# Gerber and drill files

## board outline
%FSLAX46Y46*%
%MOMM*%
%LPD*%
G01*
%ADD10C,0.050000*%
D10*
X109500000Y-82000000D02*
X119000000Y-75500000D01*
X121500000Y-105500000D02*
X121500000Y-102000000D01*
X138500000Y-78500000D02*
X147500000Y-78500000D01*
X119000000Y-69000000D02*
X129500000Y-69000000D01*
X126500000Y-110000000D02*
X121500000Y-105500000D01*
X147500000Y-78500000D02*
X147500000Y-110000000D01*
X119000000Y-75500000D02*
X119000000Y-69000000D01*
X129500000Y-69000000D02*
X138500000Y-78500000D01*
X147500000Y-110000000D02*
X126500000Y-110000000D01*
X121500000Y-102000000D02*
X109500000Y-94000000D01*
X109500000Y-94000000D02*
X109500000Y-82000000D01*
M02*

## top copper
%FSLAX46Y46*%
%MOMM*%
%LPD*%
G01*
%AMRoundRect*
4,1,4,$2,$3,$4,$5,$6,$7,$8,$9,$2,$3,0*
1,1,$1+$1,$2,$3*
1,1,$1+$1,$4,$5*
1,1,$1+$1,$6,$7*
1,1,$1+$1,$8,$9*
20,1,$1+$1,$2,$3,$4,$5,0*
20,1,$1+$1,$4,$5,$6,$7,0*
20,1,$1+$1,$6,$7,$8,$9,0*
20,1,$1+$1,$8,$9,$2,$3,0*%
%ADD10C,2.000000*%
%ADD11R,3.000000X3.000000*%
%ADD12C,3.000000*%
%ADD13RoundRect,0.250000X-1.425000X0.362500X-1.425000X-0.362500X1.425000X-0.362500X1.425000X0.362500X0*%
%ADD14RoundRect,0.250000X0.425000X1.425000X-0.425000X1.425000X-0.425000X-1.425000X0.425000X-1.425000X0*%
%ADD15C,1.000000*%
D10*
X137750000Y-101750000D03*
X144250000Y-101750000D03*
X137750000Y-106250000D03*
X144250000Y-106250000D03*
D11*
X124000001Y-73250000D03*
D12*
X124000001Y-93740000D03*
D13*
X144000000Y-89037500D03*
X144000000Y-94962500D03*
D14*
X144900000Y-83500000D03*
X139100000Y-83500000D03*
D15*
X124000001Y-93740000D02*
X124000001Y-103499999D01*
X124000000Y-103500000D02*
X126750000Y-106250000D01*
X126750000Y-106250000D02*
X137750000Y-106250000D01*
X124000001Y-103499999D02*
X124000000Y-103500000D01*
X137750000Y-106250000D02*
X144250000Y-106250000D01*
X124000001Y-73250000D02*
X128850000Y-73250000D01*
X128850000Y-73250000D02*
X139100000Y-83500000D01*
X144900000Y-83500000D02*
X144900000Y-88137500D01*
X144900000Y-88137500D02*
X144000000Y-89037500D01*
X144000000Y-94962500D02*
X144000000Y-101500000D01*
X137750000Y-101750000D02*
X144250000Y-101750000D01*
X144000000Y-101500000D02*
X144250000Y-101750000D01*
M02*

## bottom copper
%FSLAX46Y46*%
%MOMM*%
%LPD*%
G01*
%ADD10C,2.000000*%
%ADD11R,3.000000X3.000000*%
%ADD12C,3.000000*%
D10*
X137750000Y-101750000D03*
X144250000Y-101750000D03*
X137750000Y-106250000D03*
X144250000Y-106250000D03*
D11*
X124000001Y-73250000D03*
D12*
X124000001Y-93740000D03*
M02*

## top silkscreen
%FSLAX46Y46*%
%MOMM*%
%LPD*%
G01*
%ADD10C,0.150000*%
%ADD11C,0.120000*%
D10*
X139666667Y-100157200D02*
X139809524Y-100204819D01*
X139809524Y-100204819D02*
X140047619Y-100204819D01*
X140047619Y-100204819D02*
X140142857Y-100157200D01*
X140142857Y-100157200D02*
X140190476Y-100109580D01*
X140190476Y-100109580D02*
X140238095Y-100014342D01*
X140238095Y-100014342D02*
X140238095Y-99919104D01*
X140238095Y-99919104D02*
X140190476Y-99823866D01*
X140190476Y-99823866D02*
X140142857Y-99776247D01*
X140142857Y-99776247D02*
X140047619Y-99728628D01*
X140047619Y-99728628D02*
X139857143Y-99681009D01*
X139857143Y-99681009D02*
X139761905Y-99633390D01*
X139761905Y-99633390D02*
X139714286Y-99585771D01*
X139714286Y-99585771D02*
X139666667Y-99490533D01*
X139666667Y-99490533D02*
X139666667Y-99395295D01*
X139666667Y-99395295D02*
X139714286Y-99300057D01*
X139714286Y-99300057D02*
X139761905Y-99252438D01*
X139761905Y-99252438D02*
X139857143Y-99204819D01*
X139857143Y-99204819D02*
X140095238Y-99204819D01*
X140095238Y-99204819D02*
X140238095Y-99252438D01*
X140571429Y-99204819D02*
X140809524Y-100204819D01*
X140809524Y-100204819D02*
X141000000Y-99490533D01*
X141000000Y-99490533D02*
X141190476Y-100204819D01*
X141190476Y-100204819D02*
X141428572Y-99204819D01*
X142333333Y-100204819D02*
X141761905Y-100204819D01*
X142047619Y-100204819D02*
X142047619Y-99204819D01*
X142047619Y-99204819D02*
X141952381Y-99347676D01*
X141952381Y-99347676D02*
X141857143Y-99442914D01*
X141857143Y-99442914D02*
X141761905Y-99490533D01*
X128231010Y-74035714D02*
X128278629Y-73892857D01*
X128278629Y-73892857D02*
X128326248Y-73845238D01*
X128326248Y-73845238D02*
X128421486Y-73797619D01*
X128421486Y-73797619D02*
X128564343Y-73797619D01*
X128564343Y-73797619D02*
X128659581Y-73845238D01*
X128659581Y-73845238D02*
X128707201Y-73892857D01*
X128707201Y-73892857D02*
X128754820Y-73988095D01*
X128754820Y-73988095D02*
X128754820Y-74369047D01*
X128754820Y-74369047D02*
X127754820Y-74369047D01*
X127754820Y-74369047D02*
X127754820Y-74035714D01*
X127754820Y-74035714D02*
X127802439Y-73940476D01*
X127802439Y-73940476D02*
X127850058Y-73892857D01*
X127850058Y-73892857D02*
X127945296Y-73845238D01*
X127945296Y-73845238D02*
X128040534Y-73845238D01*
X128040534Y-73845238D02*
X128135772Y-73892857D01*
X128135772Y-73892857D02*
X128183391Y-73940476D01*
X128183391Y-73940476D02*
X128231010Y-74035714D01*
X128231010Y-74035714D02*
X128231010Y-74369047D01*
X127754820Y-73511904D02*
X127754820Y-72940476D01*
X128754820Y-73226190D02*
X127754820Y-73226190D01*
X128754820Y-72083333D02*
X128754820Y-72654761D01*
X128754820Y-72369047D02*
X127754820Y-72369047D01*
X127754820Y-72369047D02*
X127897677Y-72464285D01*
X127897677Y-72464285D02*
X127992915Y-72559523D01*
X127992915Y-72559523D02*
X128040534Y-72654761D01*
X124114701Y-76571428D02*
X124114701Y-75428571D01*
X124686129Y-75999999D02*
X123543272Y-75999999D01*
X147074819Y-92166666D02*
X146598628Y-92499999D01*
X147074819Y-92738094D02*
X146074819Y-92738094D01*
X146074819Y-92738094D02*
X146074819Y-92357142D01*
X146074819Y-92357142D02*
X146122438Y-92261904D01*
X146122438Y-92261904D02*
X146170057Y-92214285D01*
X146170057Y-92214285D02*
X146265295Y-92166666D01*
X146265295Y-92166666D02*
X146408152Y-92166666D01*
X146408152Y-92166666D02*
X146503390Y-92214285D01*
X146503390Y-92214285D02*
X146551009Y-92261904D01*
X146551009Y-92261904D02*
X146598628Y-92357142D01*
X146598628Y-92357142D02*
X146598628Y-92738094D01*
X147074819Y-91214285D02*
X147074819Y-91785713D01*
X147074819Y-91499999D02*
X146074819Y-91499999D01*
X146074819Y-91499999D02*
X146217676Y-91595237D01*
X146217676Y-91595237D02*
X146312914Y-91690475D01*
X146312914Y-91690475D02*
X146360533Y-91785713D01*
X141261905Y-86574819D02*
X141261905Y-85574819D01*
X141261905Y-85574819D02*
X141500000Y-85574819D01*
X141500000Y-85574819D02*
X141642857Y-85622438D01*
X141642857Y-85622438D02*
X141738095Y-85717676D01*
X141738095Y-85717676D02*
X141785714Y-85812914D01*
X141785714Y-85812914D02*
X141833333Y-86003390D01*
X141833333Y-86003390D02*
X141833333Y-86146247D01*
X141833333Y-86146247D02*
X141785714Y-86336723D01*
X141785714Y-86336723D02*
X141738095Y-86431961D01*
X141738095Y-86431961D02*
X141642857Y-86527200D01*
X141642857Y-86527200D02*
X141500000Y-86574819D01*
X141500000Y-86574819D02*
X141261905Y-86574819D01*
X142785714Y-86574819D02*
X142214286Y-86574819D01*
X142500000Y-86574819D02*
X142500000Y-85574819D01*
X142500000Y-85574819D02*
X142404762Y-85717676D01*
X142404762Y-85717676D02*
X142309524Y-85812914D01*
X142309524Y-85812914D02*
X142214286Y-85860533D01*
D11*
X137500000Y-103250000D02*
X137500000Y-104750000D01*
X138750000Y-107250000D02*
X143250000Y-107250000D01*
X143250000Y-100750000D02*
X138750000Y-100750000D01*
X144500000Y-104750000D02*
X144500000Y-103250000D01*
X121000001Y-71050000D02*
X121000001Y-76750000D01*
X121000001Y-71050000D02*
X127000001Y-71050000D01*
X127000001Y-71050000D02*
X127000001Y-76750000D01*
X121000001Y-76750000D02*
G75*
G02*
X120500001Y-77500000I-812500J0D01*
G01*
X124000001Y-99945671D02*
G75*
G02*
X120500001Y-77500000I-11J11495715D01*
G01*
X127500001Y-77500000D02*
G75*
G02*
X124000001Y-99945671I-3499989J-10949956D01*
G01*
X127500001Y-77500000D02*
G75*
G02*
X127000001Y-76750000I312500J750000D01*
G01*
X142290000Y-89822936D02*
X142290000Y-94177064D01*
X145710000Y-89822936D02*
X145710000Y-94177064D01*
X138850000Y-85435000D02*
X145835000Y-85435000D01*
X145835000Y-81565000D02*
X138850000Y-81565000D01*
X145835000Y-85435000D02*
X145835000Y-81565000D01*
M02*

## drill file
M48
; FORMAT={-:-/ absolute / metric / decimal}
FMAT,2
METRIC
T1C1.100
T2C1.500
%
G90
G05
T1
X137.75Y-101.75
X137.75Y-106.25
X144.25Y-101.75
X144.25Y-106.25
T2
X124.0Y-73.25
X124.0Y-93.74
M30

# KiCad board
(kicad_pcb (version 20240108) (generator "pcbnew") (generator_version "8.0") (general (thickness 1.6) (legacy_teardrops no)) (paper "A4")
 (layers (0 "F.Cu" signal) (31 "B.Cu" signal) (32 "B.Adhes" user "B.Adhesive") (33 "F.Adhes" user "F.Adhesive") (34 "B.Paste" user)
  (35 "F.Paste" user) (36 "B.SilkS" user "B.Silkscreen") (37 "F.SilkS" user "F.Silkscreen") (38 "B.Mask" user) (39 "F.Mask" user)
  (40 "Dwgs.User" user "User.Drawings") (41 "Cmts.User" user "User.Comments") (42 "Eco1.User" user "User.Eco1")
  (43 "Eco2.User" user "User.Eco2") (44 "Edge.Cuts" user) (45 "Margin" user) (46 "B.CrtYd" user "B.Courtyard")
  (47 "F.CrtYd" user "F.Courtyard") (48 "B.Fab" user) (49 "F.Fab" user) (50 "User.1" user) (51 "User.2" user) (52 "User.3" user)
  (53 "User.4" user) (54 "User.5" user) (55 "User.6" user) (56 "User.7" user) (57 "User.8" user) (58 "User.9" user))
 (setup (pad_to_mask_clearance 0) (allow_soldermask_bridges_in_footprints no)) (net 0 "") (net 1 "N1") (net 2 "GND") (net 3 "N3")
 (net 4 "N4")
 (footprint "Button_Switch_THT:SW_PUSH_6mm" (layer "F.Cu") (at 137.75 101.75)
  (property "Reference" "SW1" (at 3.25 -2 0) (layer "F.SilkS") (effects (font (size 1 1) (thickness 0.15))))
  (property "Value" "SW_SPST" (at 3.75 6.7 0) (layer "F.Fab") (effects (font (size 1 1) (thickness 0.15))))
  (fp_line (start -0.25 1.5) (end -0.25 3) (stroke (width 0.12) (type solid)) (layer "F.SilkS"))
  (fp_line (start 1 5.5) (end 5.5 5.5) (stroke (width 0.12) (type solid)) (layer "F.SilkS"))
  (fp_line (start 5.5 -1) (end 1 -1) (stroke (width 0.12) (type solid)) (layer "F.SilkS"))
  (fp_line (start 6.75 3) (end 6.75 1.5) (stroke (width 0.12) (type solid)) (layer "F.SilkS"))
  (pad "1" thru_hole circle (at 0 0 90) (size 2 2) (drill 1.1) (layers "*.Cu" "*.Mask") (remove_unused_layers no) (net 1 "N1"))
  (pad "1" thru_hole circle (at 6.5 0 90) (size 2 2) (drill 1.1) (layers "*.Cu" "*.Mask") (remove_unused_layers no) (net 1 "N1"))
  (pad "2" thru_hole circle (at 0 4.5 90) (size 2 2) (drill 1.1) (layers "*.Cu" "*.Mask") (remove_unused_layers no) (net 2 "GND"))
  (pad "2" thru_hole circle (at 6.5 4.5 90) (size 2 2) (drill 1.1) (layers "*.Cu" "*.Mask") (remove_unused_layers no) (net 2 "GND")))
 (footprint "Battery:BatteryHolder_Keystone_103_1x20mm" (layer "F.Cu") (at 124.000001 73.25 -90)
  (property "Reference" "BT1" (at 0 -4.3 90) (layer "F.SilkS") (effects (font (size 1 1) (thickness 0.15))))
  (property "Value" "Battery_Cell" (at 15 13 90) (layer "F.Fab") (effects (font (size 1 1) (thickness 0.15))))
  (fp_line (start -2.2 3) (end 3.5 3) (stroke (width 0.12) (type solid)) (layer "F.SilkS"))
  (fp_line (start -2.2 3) (end -2.2 -3) (stroke (width 0.12) (type solid)) (layer "F.SilkS"))
  (fp_line (start -2.2 -3) (end 3.5 -3) (stroke (width 0.12) (type solid)) (layer "F.SilkS"))
  (fp_arc (start 3.5 3) (mid 3.950694 3.136459) (end 4.25 3.5) (stroke (width 0.12) (type solid)) (layer "F.SilkS"))
  (fp_arc (start 26.695671 0) (mid 16.971103 11.358466) (end 4.25 3.5) (stroke (width 0.12) (type solid)) (layer "F.SilkS"))
  (fp_arc (start 4.25 -3.5) (mid 16.971103 -11.358466) (end 26.695671 0) (stroke (width 0.12) (type solid)) (layer "F.SilkS"))
  (fp_arc (start 4.25 -3.5) (mid 3.950694 -3.136459) (end 3.5 -3) (stroke (width 0.12) (type solid)) (layer "F.SilkS"))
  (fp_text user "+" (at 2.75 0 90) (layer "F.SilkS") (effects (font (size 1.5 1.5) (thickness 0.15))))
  (pad "1" thru_hole rect (at 0 0 270) (size 3 3) (drill 1.5) (layers "*.Cu" "*.Mask") (remove_unused_layers no) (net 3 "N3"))
  (pad "2" thru_hole circle (at 20.49 0 270) (size 3 3) (drill 1.5) (layers "*.Cu" "*.Mask") (remove_unused_layers no) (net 2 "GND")))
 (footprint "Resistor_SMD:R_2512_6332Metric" (layer "F.Cu") (at 144 92 -90)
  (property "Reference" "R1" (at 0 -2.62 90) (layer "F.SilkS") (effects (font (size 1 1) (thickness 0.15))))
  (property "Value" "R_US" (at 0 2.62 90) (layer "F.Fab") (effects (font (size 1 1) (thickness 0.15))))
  (fp_line (start -2.177064 1.71) (end 2.177064 1.71) (stroke (width 0.12) (type solid)) (layer "F.SilkS"))
  (fp_line (start -2.177064 -1.71) (end 2.177064 -1.71) (stroke (width 0.12) (type solid)) (layer "F.SilkS"))
  (pad "1" smd roundrect (at -2.9625 0 270) (size 1.225 3.35) (layers "F.Cu" "F.Paste" "F.Mask") (roundrect_rratio 0.204082) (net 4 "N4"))
  (pad "2" smd roundrect (at 2.9625 0 270) (size 1.225 3.35) (layers "F.Cu" "F.Paste" "F.Mask") (roundrect_rratio 0.204082) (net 1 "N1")))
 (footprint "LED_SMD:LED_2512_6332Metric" (layer "F.Cu") (at 142 83.5 180)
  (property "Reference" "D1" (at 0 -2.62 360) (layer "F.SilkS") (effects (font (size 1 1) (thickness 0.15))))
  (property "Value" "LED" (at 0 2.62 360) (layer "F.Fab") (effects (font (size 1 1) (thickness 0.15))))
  (fp_line (start 3.15 -1.935) (end -3.835 -1.935) (stroke (width 0.12) (type solid)) (layer "F.SilkS"))
  (fp_line (start -3.835 1.935) (end 3.15 1.935) (stroke (width 0.12) (type solid)) (layer "F.SilkS"))
  (fp_line (start -3.835 -1.935) (end -3.835 1.935) (stroke (width 0.12) (type solid)) (layer "F.SilkS"))
  (pad "1" smd roundrect (at -2.9 0 180) (size 1.35 3.35) (layers "F.Cu" "F.Paste" "F.Mask") (roundrect_rratio 0.185185) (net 4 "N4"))
  (pad "2" smd roundrect (at 2.9 0 180) (size 1.35 3.35) (layers "F.Cu" "F.Paste" "F.Mask") (roundrect_rratio 0.185185) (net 3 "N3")))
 (gr_line (start 109.5 82) (end 119 75.5) (stroke (width 0.05) (type default)) (layer "Edge.Cuts"))
 (gr_line (start 121.5 105.5) (end 121.5 102) (stroke (width 0.05) (type default)) (layer "Edge.Cuts"))
 (gr_line (start 138.5 78.5) (end 147.5 78.5) (stroke (width 0.05) (type default)) (layer "Edge.Cuts"))
 (gr_line (start 119 69) (end 129.5 69) (stroke (width 0.05) (type default)) (layer "Edge.Cuts"))
 (gr_line (start 126.5 110) (end 121.5 105.5) (stroke (width 0.05) (type default)) (layer "Edge.Cuts"))
 (gr_line (start 147.5 78.5) (end 147.5 110) (stroke (width 0.05) (type default)) (layer "Edge.Cuts"))
 (gr_line (start 119 75.5) (end 119 69) (stroke (width 0.05) (type default)) (layer "Edge.Cuts"))
 (gr_line (start 129.5 69) (end 138.5 78.5) (stroke (width 0.05) (type default)) (layer "Edge.Cuts"))
 (gr_line (start 147.5 110) (end 126.5 110) (stroke (width 0.05) (type default)) (layer "Edge.Cuts"))
 (gr_line (start 121.5 102) (end 109.5 94) (stroke (width 0.05) (type default)) (layer "Edge.Cuts"))
 (gr_line (start 109.5 94) (end 109.5 82) (stroke (width 0.05) (type default)) (layer "Edge.Cuts"))
 (segment (start 124.000001 93.74) (end 124.000001 103.499999) (width 1) (layer "F.Cu") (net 2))
 (segment (start 124 103.5) (end 126.75 106.25) (width 1) (layer "F.Cu") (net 2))
 (segment (start 126.75 106.25) (end 137.75 106.25) (width 1) (layer "F.Cu") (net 2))
 (segment (start 124.000001 103.499999) (end 124 103.5) (width 1) (layer "F.Cu") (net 2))
 (segment (start 137.75 106.25) (end 144.25 106.25) (width 1) (layer "F.Cu") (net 2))
 (segment (start 124.000001 73.25) (end 128.85 73.25) (width 1) (layer "F.Cu") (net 3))
 (segment (start 128.85 73.25) (end 139.1 83.5) (width 1) (layer "F.Cu") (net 3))
 (segment (start 144.9 83.5) (end 144.9 88.1375) (width 1) (layer "F.Cu") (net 4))
 (segment (start 144.9 88.1375) (end 144 89.0375) (width 1) (layer "F.Cu") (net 4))
 (segment (start 144 94.9625) (end 144 101.5) (width 1) (layer "F.Cu") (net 1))
 (segment (start 137.75 101.75) (end 144.25 101.75) (width 1) (layer "F.Cu") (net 1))
 (segment (start 144 101.5) (end 144.25 101.75) (width 1) (layer "F.Cu") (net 1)))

